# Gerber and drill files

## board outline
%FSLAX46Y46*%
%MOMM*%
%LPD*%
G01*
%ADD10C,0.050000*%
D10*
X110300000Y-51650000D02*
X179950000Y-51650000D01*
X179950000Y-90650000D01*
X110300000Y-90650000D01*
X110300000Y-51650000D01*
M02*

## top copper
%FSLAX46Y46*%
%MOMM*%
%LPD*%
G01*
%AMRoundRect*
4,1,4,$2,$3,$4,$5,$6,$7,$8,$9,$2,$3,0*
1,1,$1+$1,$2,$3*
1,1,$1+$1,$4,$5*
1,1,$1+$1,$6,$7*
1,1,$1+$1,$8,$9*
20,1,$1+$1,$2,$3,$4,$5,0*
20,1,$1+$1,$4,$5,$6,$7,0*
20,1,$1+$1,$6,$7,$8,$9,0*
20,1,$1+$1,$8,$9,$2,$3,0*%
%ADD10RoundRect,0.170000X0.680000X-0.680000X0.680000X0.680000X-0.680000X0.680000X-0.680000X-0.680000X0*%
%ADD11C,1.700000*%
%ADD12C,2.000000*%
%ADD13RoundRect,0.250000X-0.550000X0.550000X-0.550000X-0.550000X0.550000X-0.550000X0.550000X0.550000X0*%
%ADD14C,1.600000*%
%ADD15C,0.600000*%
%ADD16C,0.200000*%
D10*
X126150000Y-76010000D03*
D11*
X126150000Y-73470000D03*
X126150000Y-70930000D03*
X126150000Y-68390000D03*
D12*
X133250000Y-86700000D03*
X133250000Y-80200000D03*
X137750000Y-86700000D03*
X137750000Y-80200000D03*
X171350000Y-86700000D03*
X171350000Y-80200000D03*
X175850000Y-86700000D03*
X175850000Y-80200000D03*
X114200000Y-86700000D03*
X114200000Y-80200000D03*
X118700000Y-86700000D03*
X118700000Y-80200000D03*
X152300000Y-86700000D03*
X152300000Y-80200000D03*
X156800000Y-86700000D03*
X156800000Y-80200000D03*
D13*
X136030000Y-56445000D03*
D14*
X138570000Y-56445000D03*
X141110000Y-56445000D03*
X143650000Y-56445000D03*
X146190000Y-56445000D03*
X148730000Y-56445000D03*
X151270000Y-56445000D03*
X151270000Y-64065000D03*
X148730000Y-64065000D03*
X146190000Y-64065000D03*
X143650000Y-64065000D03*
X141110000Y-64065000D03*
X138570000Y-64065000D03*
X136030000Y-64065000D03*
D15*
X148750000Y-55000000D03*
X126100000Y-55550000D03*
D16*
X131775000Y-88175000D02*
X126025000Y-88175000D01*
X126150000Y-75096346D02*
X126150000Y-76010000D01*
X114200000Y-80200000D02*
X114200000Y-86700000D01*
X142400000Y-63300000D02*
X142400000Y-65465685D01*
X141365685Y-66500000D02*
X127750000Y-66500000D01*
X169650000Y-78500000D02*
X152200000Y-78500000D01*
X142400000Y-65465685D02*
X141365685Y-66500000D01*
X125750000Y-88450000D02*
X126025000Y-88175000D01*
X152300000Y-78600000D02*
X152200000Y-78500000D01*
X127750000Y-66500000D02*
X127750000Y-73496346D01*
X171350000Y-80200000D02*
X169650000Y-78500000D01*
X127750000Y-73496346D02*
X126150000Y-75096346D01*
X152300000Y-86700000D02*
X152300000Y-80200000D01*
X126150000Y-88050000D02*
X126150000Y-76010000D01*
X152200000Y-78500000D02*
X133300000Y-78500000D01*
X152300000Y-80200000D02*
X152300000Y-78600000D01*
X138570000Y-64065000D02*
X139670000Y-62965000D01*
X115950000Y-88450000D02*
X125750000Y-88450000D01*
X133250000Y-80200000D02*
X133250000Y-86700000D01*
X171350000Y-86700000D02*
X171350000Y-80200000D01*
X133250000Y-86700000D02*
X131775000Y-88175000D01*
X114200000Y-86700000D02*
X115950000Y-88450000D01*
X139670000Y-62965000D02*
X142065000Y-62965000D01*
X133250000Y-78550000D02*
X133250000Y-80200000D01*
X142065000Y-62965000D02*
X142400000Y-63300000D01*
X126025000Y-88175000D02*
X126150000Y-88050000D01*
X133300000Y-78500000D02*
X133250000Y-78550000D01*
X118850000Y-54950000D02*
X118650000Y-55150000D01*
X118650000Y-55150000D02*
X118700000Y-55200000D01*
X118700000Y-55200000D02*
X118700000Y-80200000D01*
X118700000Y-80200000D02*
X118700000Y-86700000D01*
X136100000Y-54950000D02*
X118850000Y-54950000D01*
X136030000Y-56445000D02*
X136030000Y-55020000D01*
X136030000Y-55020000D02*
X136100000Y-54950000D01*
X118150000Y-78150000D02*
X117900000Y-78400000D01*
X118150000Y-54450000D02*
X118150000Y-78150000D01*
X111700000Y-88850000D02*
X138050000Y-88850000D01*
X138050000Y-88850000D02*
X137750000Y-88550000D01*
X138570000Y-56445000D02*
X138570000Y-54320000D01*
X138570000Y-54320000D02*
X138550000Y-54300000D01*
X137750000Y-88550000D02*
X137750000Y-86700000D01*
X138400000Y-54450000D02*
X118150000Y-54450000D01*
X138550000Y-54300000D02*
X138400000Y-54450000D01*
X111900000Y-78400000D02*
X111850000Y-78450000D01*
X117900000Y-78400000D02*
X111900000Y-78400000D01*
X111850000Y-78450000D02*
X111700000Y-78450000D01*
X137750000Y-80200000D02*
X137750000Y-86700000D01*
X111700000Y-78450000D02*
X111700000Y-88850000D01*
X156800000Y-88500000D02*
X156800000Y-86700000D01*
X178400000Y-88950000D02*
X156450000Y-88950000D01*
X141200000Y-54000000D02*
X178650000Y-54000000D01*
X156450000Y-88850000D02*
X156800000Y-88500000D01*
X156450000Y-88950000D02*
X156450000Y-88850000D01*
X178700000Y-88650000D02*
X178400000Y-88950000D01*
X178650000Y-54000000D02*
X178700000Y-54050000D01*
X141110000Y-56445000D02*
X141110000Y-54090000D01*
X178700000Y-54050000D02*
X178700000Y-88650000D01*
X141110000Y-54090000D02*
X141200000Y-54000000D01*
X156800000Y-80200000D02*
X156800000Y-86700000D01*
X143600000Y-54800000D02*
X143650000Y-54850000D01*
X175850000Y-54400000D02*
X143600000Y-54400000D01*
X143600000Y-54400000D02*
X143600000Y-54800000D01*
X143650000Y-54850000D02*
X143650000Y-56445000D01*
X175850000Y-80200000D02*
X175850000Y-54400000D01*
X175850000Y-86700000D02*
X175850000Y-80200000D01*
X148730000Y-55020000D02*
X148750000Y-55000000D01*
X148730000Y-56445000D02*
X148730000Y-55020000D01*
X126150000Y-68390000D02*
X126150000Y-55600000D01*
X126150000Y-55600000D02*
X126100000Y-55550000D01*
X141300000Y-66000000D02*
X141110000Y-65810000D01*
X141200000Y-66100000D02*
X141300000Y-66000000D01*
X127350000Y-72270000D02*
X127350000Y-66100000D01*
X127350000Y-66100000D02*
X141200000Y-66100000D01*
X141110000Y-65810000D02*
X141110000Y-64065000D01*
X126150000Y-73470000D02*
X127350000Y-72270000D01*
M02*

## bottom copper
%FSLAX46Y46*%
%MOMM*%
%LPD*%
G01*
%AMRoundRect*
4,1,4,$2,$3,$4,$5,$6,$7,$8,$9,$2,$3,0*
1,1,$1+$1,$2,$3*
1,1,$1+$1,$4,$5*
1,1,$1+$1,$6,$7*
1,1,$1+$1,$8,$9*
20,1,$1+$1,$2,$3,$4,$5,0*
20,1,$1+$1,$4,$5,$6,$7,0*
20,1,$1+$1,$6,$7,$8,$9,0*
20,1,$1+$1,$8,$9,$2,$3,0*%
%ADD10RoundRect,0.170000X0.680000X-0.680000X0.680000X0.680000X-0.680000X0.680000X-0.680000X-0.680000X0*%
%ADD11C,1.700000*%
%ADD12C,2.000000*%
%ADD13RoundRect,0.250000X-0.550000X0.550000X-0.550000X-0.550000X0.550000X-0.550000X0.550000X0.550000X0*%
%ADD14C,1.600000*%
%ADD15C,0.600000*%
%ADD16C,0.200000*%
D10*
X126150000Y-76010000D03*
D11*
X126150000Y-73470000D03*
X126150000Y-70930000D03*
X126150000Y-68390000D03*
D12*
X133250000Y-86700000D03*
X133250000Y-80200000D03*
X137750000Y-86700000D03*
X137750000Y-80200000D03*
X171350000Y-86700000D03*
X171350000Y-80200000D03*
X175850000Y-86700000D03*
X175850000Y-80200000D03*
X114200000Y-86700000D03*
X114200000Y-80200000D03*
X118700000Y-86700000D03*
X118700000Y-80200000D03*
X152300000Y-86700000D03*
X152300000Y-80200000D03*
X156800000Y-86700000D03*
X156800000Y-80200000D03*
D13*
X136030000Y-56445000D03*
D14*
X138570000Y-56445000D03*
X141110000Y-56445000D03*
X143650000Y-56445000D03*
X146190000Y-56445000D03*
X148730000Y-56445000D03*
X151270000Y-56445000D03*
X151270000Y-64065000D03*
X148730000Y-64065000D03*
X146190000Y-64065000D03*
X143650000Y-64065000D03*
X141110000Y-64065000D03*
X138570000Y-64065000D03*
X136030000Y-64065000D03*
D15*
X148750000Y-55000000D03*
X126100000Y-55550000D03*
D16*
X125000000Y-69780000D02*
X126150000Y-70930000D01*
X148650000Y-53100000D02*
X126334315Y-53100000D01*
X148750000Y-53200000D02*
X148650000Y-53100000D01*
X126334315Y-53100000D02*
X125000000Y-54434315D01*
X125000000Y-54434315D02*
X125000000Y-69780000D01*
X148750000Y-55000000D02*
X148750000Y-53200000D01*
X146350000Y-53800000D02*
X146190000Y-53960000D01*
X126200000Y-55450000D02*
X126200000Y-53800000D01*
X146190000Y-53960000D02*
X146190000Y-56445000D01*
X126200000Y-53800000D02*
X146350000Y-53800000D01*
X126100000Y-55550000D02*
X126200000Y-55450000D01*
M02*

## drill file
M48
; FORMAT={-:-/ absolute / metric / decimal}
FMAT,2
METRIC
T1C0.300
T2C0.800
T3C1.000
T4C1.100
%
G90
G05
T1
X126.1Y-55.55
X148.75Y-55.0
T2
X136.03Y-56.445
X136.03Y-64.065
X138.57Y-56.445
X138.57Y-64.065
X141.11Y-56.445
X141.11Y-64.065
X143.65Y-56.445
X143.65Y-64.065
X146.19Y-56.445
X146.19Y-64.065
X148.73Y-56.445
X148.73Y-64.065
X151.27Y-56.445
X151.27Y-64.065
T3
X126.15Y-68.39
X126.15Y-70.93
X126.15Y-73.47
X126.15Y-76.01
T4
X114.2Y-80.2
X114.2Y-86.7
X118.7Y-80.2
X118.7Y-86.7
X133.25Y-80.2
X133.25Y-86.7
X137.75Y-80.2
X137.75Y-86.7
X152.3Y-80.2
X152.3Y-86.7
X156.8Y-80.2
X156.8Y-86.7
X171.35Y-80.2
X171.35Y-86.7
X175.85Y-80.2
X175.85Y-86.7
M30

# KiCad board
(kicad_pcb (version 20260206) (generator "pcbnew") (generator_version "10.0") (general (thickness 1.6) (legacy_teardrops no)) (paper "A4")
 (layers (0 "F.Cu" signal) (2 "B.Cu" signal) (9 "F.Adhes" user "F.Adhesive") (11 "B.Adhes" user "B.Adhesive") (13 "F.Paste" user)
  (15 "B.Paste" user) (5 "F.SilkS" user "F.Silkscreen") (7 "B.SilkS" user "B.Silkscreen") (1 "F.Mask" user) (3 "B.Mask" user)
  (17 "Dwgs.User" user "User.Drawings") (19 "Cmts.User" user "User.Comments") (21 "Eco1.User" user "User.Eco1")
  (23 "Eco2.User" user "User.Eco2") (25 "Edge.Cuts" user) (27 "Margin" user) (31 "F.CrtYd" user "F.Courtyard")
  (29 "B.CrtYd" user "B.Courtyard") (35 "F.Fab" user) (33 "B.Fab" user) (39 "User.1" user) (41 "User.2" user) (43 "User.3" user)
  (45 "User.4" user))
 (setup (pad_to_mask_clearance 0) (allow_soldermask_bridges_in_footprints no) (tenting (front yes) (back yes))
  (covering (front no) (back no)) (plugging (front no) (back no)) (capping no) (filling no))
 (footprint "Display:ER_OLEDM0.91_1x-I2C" (layer "F.Cu") (at 126.15 76.01 90)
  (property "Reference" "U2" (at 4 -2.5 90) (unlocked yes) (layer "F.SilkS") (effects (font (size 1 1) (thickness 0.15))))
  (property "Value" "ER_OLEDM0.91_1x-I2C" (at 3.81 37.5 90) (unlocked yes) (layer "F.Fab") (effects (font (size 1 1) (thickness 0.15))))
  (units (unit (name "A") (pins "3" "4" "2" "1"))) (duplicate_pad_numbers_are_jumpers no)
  (pad "1" thru_hole roundrect (at 0 0 90) (size 1.7 1.7) (drill 1) (layers "*.Cu" "*.Mask") (remove_unused_layers no)
   (roundrect_rratio 0.1) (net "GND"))
  (pad "2" thru_hole circle (at 2.54 0 90) (size 1.7 1.7) (drill 1) (layers "*.Cu" "*.Mask") (remove_unused_layers no) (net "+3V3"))
  (pad "3" thru_hole circle (at 5.08 0 90) (size 1.7 1.7) (drill 1) (layers "*.Cu" "*.Mask") (remove_unused_layers no) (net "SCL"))
  (pad "4" thru_hole circle (at 7.62 0 90) (size 1.7 1.7) (drill 1) (layers "*.Cu" "*.Mask") (remove_unused_layers no) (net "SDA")))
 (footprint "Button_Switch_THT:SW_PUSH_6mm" (layer "F.Cu") (at 133.25 86.7 90)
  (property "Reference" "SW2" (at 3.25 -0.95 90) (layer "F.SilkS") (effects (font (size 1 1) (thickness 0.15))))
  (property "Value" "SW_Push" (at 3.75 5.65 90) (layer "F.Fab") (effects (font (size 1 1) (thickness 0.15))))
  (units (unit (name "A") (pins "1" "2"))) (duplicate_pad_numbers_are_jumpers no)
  (pad "1" thru_hole circle (at 0 0 180) (size 2 2) (drill 1.1) (layers "*.Cu" "*.Mask") (remove_unused_layers no) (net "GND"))
  (pad "1" thru_hole circle (at 6.5 0 180) (size 2 2) (drill 1.1) (layers "*.Cu" "*.Mask") (remove_unused_layers no) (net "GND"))
  (pad "2" thru_hole circle (at 0 4.5 180) (size 2 2) (drill 1.1) (layers "*.Cu" "*.Mask") (remove_unused_layers no) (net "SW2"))
  (pad "2" thru_hole circle (at 6.5 4.5 180) (size 2 2) (drill 1.1) (layers "*.Cu" "*.Mask") (remove_unused_layers no) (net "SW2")))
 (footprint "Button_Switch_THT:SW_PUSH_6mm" (layer "F.Cu") (at 171.35 86.7 90)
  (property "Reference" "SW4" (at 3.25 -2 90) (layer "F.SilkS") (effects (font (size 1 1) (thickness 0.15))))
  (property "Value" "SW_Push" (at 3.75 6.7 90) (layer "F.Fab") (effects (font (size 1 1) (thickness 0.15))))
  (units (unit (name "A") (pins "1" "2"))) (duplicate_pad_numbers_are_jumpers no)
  (pad "1" thru_hole circle (at 0 0 180) (size 2 2) (drill 1.1) (layers "*.Cu" "*.Mask") (remove_unused_layers no) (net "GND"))
  (pad "1" thru_hole circle (at 6.5 0 180) (size 2 2) (drill 1.1) (layers "*.Cu" "*.Mask") (remove_unused_layers no) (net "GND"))
  (pad "2" thru_hole circle (at 0 4.5 180) (size 2 2) (drill 1.1) (layers "*.Cu" "*.Mask") (remove_unused_layers no) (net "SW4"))
  (pad "2" thru_hole circle (at 6.5 4.5 180) (size 2 2) (drill 1.1) (layers "*.Cu" "*.Mask") (remove_unused_layers no) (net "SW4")))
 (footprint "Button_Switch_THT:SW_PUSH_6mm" (layer "F.Cu") (at 114.2 86.7 90)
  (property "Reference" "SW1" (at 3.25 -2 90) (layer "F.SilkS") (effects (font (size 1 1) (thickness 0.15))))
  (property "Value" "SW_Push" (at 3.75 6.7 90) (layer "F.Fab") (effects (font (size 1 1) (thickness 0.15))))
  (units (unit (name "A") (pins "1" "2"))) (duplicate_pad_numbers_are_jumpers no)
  (pad "1" thru_hole circle (at 0 0 180) (size 2 2) (drill 1.1) (layers "*.Cu" "*.Mask") (remove_unused_layers no) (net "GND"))
  (pad "1" thru_hole circle (at 6.5 0 180) (size 2 2) (drill 1.1) (layers "*.Cu" "*.Mask") (remove_unused_layers no) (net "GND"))
  (pad "2" thru_hole circle (at 0 4.5 180) (size 2 2) (drill 1.1) (layers "*.Cu" "*.Mask") (remove_unused_layers no) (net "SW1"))
  (pad "2" thru_hole circle (at 6.5 4.5 180) (size 2 2) (drill 1.1) (layers "*.Cu" "*.Mask") (remove_unused_layers no) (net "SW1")))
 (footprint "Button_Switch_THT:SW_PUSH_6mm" (layer "F.Cu") (at 152.3 86.7 90)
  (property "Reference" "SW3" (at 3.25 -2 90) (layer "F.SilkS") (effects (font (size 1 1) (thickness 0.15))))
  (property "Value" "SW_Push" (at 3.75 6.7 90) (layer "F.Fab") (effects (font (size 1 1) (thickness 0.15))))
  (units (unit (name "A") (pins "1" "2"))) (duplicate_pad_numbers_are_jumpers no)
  (pad "1" thru_hole circle (at 0 0 180) (size 2 2) (drill 1.1) (layers "*.Cu" "*.Mask") (remove_unused_layers no) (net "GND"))
  (pad "1" thru_hole circle (at 6.5 0 180) (size 2 2) (drill 1.1) (layers "*.Cu" "*.Mask") (remove_unused_layers no) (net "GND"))
  (pad "2" thru_hole circle (at 0 4.5 180) (size 2 2) (drill 1.1) (layers "*.Cu" "*.Mask") (remove_unused_layers no) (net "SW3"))
  (pad "2" thru_hole circle (at 6.5 4.5 180) (size 2 2) (drill 1.1) (layers "*.Cu" "*.Mask") (remove_unused_layers no) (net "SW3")))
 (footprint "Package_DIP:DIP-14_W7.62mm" (layer "B.Cu") (at 136.03 56.445 -90)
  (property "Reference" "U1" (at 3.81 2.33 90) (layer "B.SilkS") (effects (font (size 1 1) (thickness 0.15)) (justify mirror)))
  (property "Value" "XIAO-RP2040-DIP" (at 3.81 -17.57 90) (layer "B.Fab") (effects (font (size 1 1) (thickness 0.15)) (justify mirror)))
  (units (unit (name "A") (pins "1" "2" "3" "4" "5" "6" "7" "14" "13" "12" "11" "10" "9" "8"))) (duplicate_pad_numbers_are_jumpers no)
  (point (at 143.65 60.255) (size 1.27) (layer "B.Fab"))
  (pad "1" thru_hole roundrect (at 0 0 270) (size 1.6 1.6) (drill 0.8) (layers "*.Cu" "*.Mask") (remove_unused_layers no)
   (roundrect_rratio 0.15625) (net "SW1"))
  (pad "2" thru_hole circle (at 0 -2.54 270) (size 1.6 1.6) (drill 0.8) (layers "*.Cu" "*.Mask") (remove_unused_layers no) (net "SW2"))
  (pad "3" thru_hole circle (at 0 -5.08 270) (size 1.6 1.6) (drill 0.8) (layers "*.Cu" "*.Mask") (remove_unused_layers no) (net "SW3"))
  (pad "4" thru_hole circle (at 0 -7.62 270) (size 1.6 1.6) (drill 0.8) (layers "*.Cu" "*.Mask") (remove_unused_layers no) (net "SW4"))
  (pad "5" thru_hole circle (at 0 -10.16 270) (size 1.6 1.6) (drill 0.8) (layers "*.Cu" "*.Mask") (remove_unused_layers no) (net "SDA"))
  (pad "6" thru_hole circle (at 0 -12.7 270) (size 1.6 1.6) (drill 0.8) (layers "*.Cu" "*.Mask") (remove_unused_layers no) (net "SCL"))
  (pad "7" thru_hole circle (at 0 -15.24 270) (size 1.6 1.6) (drill 0.8) (layers "*.Cu" "*.Mask") (remove_unused_layers no)
   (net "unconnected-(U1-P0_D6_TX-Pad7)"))
  (pad "8" thru_hole circle (at 7.62 -15.24 270) (size 1.6 1.6) (drill 0.8) (layers "*.Cu" "*.Mask") (remove_unused_layers no))
  (pad "9" thru_hole circle (at 7.62 -12.7 270) (size 1.6 1.6) (drill 0.8) (layers "*.Cu" "*.Mask") (remove_unused_layers no))
  (pad "10" thru_hole circle (at 7.62 -10.16 270) (size 1.6 1.6) (drill 0.8) (layers "*.Cu" "*.Mask") (remove_unused_layers no))
  (pad "11" thru_hole circle (at 7.62 -7.62 270) (size 1.6 1.6) (drill 0.8) (layers "*.Cu" "*.Mask") (remove_unused_layers no))
  (pad "12" thru_hole circle (at 7.62 -5.08 270) (size 1.6 1.6) (drill 0.8) (layers "*.Cu" "*.Mask") (remove_unused_layers no) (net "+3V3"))
  (pad "13" thru_hole circle (at 7.62 -2.54 270) (size 1.6 1.6) (drill 0.8) (layers "*.Cu" "*.Mask") (remove_unused_layers no) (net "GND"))
  (pad "14" thru_hole circle (at 7.62 0 270) (size 1.6 1.6) (drill 0.8) (layers "*.Cu" "*.Mask") (remove_unused_layers no)))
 (gr_rect (start 110.3 51.65) (end 179.95 90.65) (stroke (width 0.05) (type default)) (fill no) (layer "Edge.Cuts"))
 (segment (start 131.775 88.175) (end 126.025 88.175) (width 0.2) (layer "F.Cu") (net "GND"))
 (segment (start 126.15 75.096346) (end 126.15 76.01) (width 0.2) (layer "F.Cu") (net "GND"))
 (segment (start 114.2 80.2) (end 114.2 86.7) (width 0.2) (layer "F.Cu") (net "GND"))
 (segment (start 142.4 63.3) (end 142.4 65.465685) (width 0.2) (layer "F.Cu") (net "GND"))
 (segment (start 141.365685 66.5) (end 127.75 66.5) (width 0.2) (layer "F.Cu") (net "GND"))
 (segment (start 169.65 78.5) (end 152.2 78.5) (width 0.2) (layer "F.Cu") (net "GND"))
 (segment (start 142.4 65.465685) (end 141.365685 66.5) (width 0.2) (layer "F.Cu") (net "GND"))
 (segment (start 125.75 88.45) (end 126.025 88.175) (width 0.2) (layer "F.Cu") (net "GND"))
 (segment (start 152.3 78.6) (end 152.2 78.5) (width 0.2) (layer "F.Cu") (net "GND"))
 (segment (start 127.75 66.5) (end 127.75 73.496346) (width 0.2) (layer "F.Cu") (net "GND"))
 (segment (start 171.35 80.2) (end 169.65 78.5) (width 0.2) (layer "F.Cu") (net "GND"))
 (segment (start 127.75 73.496346) (end 126.15 75.096346) (width 0.2) (layer "F.Cu") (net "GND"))
 (segment (start 152.3 86.7) (end 152.3 80.2) (width 0.2) (layer "F.Cu") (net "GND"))
 (segment (start 126.15 88.05) (end 126.15 76.01) (width 0.2) (layer "F.Cu") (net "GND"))
 (segment (start 152.2 78.5) (end 133.3 78.5) (width 0.2) (layer "F.Cu") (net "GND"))
 (segment (start 152.3 80.2) (end 152.3 78.6) (width 0.2) (layer "F.Cu") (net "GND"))
 (segment (start 138.57 64.065) (end 139.67 62.965) (width 0.2) (layer "F.Cu") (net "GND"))
 (segment (start 115.95 88.45) (end 125.75 88.45) (width 0.2) (layer "F.Cu") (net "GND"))
 (segment (start 133.25 80.2) (end 133.25 86.7) (width 0.2) (layer "F.Cu") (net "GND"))
 (segment (start 171.35 86.7) (end 171.35 80.2) (width 0.2) (layer "F.Cu") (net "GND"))
 (segment (start 133.25 86.7) (end 131.775 88.175) (width 0.2) (layer "F.Cu") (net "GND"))
 (segment (start 114.2 86.7) (end 115.95 88.45) (width 0.2) (layer "F.Cu") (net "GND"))
 (segment (start 139.67 62.965) (end 142.065 62.965) (width 0.2) (layer "F.Cu") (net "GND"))
 (segment (start 133.25 78.55) (end 133.25 80.2) (width 0.2) (layer "F.Cu") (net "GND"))
 (segment (start 142.065 62.965) (end 142.4 63.3) (width 0.2) (layer "F.Cu") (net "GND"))
 (segment (start 126.025 88.175) (end 126.15 88.05) (width 0.2) (layer "F.Cu") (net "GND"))
 (segment (start 133.3 78.5) (end 133.25 78.55) (width 0.2) (layer "F.Cu") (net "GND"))
 (segment (start 118.85 54.95) (end 118.65 55.15) (width 0.2) (layer "F.Cu") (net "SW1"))
 (segment (start 118.65 55.15) (end 118.7 55.2) (width 0.2) (layer "F.Cu") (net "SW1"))
 (segment (start 118.7 55.2) (end 118.7 80.2) (width 0.2) (layer "F.Cu") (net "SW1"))
 (segment (start 118.7 80.2) (end 118.7 86.7) (width 0.2) (layer "F.Cu") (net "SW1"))
 (segment (start 136.1 54.95) (end 118.85 54.95) (width 0.2) (layer "F.Cu") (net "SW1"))
 (segment (start 136.03 56.445) (end 136.03 55.02) (width 0.2) (layer "F.Cu") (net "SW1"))
 (segment (start 136.03 55.02) (end 136.1 54.95) (width 0.2) (layer "F.Cu") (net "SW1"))
 (segment (start 118.15 78.15) (end 117.9 78.4) (width 0.2) (layer "F.Cu") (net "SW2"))
 (segment (start 118.15 54.45) (end 118.15 78.15) (width 0.2) (layer "F.Cu") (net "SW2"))
 (segment (start 111.7 88.85) (end 138.05 88.85) (width 0.2) (layer "F.Cu") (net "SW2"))
 (segment (start 138.05 88.85) (end 137.75 88.55) (width 0.2) (layer "F.Cu") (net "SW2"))
 (segment (start 138.57 56.445) (end 138.57 54.32) (width 0.2) (layer "F.Cu") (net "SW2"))
 (segment (start 138.57 54.32) (end 138.55 54.3) (width 0.2) (layer "F.Cu") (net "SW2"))
 (segment (start 137.75 88.55) (end 137.75 86.7) (width 0.2) (layer "F.Cu") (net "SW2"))
 (segment (start 138.4 54.45) (end 118.15 54.45) (width 0.2) (layer "F.Cu") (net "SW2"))
 (segment (start 138.55 54.3) (end 138.4 54.45) (width 0.2) (layer "F.Cu") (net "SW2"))
 (segment (start 111.9 78.4) (end 111.85 78.45) (width 0.2) (layer "F.Cu") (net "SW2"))
 (segment (start 117.9 78.4) (end 111.9 78.4) (width 0.2) (layer "F.Cu") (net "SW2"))
 (segment (start 111.85 78.45) (end 111.7 78.45) (width 0.2) (layer "F.Cu") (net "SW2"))
 (segment (start 137.75 80.2) (end 137.75 86.7) (width 0.2) (layer "F.Cu") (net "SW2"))
 (segment (start 111.7 78.45) (end 111.7 88.85) (width 0.2) (layer "F.Cu") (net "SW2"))
 (segment (start 156.8 88.5) (end 156.8 86.7) (width 0.2) (layer "F.Cu") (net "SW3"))
 (segment (start 178.4 88.95) (end 156.45 88.95) (width 0.2) (layer "F.Cu") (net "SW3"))
 (segment (start 141.2 54) (end 178.65 54) (width 0.2) (layer "F.Cu") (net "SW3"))
 (segment (start 156.45 88.85) (end 156.8 88.5) (width 0.2) (layer "F.Cu") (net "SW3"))
 (segment (start 156.45 88.95) (end 156.45 88.85) (width 0.2) (layer "F.Cu") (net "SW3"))
 (segment (start 178.7 88.65) (end 178.4 88.95) (width 0.2) (layer "F.Cu") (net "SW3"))
 (segment (start 178.65 54) (end 178.7 54.05) (width 0.2) (layer "F.Cu") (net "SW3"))
 (segment (start 141.11 56.445) (end 141.11 54.09) (width 0.2) (layer "F.Cu") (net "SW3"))
 (segment (start 178.7 54.05) (end 178.7 88.65) (width 0.2) (layer "F.Cu") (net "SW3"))
 (segment (start 141.11 54.09) (end 141.2 54) (width 0.2) (layer "F.Cu") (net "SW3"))
 (segment (start 156.8 80.2) (end 156.8 86.7) (width 0.2) (layer "F.Cu") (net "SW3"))
 (segment (start 143.6 54.8) (end 143.65 54.85) (width 0.2) (layer "F.Cu") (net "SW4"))
 (segment (start 175.85 54.4) (end 143.6 54.4) (width 0.2) (layer "F.Cu") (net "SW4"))
 (segment (start 143.6 54.4) (end 143.6 54.8) (width 0.2) (layer "F.Cu") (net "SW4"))
 (segment (start 143.65 54.85) (end 143.65 56.445) (width 0.2) (layer "F.Cu") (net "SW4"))
 (segment (start 175.85 80.2) (end 175.85 54.4) (width 0.2) (layer "F.Cu") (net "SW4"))
 (segment (start 175.85 86.7) (end 175.85 80.2) (width 0.2) (layer "F.Cu") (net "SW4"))
 (segment (start 148.73 55.02) (end 148.75 55) (width 0.2) (layer "F.Cu") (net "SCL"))
 (segment (start 148.73 56.445) (end 148.73 55.02) (width 0.2) (layer "F.Cu") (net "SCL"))
 (via (at 148.75 55) (size 0.6) (drill 0.3) (layers "F.Cu" "B.Cu") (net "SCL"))
 (segment (start 125 69.78) (end 126.15 70.93) (width 0.2) (layer "B.Cu") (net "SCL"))
 (segment (start 148.65 53.1) (end 126.334315 53.1) (width 0.2) (layer "B.Cu") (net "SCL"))
 (segment (start 148.75 53.2) (end 148.65 53.1) (width 0.2) (layer "B.Cu") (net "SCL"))
 (segment (start 126.334315 53.1) (end 125 54.434315) (width 0.2) (layer "B.Cu") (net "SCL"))
 (segment (start 125 54.434315) (end 125 69.78) (width 0.2) (layer "B.Cu") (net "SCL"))
 (segment (start 148.75 55) (end 148.75 53.2) (width 0.2) (layer "B.Cu") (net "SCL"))
 (segment (start 126.15 68.39) (end 126.15 55.6) (width 0.2) (layer "F.Cu") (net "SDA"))
 (segment (start 126.15 55.6) (end 126.1 55.55) (width 0.2) (layer "F.Cu") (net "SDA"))
 (via (at 126.1 55.55) (size 0.6) (drill 0.3) (layers "F.Cu" "B.Cu") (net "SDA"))
 (segment (start 146.35 53.8) (end 146.19 53.96) (width 0.2) (layer "B.Cu") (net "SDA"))
 (segment (start 126.2 55.45) (end 126.2 53.8) (width 0.2) (layer "B.Cu") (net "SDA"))
 (segment (start 146.19 53.96) (end 146.19 56.445) (width 0.2) (layer "B.Cu") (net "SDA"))
 (segment (start 126.2 53.8) (end 146.35 53.8) (width 0.2) (layer "B.Cu") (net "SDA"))
 (segment (start 126.1 55.55) (end 126.2 55.45) (width 0.2) (layer "B.Cu") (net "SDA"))
 (segment (start 141.3 66) (end 141.11 65.81) (width 0.2) (layer "F.Cu") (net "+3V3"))
 (segment (start 141.2 66.1) (end 141.3 66) (width 0.2) (layer "F.Cu") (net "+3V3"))
 (segment (start 127.35 72.27) (end 127.35 66.1) (width 0.2) (layer "F.Cu") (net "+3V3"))
 (segment (start 127.35 66.1) (end 141.2 66.1) (width 0.2) (layer "F.Cu") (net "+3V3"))
 (segment (start 141.11 65.81) (end 141.11 64.065) (width 0.2) (layer "F.Cu") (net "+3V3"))
 (segment (start 126.15 73.47) (end 127.35 72.27) (width 0.2) (layer "F.Cu") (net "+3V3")))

